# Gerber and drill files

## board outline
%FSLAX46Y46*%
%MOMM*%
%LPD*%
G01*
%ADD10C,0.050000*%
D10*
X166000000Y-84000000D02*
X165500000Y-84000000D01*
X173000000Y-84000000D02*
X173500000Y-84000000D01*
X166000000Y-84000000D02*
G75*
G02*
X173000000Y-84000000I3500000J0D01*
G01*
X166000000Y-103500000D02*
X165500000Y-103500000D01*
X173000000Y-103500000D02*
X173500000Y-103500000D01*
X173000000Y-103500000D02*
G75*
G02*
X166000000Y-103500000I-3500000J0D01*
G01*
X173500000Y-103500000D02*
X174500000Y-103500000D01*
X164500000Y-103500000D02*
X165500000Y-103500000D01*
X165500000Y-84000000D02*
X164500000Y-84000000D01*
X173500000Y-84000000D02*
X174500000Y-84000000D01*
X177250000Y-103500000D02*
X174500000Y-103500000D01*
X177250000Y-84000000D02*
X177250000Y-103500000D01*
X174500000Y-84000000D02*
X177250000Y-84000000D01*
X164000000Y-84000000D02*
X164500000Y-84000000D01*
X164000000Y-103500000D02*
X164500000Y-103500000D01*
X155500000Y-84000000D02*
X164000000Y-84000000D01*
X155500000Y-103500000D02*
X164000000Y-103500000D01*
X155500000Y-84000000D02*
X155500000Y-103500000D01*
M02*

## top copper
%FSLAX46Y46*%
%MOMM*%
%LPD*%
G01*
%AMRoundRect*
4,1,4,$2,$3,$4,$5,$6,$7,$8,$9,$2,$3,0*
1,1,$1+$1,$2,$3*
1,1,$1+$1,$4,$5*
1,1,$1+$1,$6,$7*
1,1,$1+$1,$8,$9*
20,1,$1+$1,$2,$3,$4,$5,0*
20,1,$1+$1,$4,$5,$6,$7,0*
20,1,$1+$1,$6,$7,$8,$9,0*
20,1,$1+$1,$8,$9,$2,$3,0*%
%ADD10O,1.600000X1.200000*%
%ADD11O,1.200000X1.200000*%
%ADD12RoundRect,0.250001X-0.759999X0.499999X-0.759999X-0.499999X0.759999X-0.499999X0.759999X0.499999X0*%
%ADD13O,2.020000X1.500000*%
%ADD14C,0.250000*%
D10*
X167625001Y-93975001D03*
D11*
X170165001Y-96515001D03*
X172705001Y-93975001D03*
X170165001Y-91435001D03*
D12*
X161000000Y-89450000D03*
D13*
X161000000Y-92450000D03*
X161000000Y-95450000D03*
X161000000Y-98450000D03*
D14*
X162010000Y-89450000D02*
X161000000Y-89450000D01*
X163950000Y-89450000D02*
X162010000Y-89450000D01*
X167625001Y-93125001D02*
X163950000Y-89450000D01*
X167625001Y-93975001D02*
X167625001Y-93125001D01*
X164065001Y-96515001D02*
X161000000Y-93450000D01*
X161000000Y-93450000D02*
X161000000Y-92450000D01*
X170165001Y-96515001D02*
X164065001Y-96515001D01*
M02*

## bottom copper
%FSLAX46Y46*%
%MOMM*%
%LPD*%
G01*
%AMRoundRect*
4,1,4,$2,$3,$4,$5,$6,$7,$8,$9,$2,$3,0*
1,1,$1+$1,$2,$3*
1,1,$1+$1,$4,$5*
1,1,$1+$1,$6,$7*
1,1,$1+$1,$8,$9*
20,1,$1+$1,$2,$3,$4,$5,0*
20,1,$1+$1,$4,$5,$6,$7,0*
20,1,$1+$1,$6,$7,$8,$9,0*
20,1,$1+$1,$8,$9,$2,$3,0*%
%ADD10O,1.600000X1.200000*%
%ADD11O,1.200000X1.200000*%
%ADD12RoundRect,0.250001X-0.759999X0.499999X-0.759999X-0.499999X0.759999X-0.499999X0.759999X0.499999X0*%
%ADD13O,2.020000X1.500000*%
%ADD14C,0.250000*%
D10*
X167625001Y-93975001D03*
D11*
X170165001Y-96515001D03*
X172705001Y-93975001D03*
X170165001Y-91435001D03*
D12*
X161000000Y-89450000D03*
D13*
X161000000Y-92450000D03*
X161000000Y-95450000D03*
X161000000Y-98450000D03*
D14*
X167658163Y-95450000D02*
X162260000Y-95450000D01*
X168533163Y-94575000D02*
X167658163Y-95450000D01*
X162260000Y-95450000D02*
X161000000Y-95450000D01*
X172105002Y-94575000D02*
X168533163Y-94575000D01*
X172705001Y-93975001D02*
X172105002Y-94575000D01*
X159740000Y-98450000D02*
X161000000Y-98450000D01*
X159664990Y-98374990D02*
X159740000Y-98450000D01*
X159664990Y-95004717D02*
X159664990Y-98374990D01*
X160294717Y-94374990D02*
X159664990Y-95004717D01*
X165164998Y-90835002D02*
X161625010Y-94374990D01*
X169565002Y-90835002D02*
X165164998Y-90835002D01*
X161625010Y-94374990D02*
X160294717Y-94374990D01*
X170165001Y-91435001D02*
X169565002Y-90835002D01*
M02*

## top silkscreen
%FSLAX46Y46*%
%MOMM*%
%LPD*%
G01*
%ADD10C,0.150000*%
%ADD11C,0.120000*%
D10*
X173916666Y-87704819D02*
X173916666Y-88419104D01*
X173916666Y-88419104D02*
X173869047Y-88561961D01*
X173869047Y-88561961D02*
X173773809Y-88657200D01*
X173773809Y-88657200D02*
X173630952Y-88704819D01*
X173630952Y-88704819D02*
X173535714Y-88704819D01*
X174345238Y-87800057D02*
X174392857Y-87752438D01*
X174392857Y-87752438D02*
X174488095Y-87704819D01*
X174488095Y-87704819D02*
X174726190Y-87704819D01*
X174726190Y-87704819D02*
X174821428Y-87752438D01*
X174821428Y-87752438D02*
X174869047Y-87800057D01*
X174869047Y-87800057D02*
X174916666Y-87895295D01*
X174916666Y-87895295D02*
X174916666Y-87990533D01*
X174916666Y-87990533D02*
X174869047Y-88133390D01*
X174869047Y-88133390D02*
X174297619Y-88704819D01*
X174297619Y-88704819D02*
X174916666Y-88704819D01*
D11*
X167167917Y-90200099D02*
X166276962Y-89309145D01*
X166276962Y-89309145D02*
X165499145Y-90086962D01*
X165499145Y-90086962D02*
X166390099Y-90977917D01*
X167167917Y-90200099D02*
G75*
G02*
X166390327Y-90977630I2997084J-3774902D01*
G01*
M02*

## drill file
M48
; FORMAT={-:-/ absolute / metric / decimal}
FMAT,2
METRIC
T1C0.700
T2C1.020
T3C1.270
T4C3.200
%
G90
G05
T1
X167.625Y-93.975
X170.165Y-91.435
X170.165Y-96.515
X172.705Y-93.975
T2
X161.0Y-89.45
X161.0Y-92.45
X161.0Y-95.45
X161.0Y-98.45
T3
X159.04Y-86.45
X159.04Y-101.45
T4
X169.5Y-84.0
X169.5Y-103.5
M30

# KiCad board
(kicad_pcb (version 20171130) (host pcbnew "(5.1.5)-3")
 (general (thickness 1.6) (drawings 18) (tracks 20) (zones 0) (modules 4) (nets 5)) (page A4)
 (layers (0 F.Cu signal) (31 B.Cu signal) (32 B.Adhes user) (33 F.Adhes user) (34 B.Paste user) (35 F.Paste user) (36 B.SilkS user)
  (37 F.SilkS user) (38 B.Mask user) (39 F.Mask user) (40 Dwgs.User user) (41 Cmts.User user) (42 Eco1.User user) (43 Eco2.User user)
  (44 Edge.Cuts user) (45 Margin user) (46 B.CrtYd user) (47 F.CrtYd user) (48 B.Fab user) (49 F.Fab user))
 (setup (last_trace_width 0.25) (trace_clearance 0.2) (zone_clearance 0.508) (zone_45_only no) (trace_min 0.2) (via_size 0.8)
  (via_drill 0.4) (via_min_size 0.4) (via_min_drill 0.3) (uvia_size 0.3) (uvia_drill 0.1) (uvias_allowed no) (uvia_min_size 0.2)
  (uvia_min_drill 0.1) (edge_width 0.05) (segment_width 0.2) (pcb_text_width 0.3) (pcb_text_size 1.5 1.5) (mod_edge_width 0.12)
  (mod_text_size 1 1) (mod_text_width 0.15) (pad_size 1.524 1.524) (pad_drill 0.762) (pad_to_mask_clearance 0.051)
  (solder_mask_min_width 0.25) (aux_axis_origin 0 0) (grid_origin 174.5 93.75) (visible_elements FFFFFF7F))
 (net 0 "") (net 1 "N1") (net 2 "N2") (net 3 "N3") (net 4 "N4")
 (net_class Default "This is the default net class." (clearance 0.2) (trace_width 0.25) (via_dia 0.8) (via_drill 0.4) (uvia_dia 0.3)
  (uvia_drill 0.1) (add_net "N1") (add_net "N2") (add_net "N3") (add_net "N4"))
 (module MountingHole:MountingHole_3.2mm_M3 (layer F.Cu) (at 169.5 84)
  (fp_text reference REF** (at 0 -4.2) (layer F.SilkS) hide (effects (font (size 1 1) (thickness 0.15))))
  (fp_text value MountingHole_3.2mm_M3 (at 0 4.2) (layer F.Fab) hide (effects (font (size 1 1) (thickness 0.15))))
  (pad 1 np_thru_hole circle (at 0 0) (size 3.2 3.2) (drill 3.2) (layers *.Cu *.Mask)))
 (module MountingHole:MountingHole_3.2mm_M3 (layer F.Cu) (at 169.5 103.5)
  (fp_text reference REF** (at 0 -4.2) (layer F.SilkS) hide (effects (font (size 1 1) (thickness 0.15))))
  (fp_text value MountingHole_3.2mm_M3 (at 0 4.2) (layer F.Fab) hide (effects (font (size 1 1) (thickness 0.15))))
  (pad 1 np_thru_hole circle (at 0 0) (size 3.2 3.2) (drill 3.2) (layers *.Cu *.Mask)))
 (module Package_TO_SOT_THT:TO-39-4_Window (layer F.Cu) (at 167.625001 93.975001)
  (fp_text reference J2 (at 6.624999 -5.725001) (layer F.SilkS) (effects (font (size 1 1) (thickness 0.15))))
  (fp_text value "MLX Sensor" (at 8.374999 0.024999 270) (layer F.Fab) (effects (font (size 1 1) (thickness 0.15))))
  (fp_line (start -0.457084 -3.774902) (end -1.348039 -4.665856) (layer F.SilkS) (width 0.12))
  (fp_line (start -1.348039 -4.665856) (end -2.125856 -3.888039) (layer F.SilkS) (width 0.12))
  (fp_line (start -2.125856 -3.888039) (end -1.234902 -2.997084) (layer F.SilkS) (width 0.12))
  (fp_arc (start 2.54 0) (end -0.457084 -3.774902) (angle 346.9) (layer F.SilkS) (width 0.12))
  (pad 1 thru_hole oval (at 0 0) (size 1.6 1.2) (drill 0.7) (layers *.Cu *.Mask) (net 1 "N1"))
  (pad 2 thru_hole oval (at 2.54 2.54) (size 1.2 1.2) (drill 0.7) (layers *.Cu *.Mask) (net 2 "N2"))
  (pad 3 thru_hole oval (at 5.08 0) (size 1.2 1.2) (drill 0.7) (layers *.Cu *.Mask) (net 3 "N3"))
  (pad 4 thru_hole oval (at 2.54 -2.54) (size 1.2 1.2) (drill 0.7) (layers *.Cu *.Mask) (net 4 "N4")))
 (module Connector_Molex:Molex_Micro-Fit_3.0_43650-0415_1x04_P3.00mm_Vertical (layer B.Cu) (at 161 89.45 270)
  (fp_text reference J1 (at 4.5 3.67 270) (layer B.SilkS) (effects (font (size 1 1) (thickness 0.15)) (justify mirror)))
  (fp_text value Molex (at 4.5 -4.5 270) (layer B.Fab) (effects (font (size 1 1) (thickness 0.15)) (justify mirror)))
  (pad "" np_thru_hole circle (at -3 1.96 270) (size 1.27 1.27) (drill 1.27) (layers *.Cu *.Mask))
  (pad "" np_thru_hole circle (at 12 1.96 270) (size 1.27 1.27) (drill 1.27) (layers *.Cu *.Mask))
  (pad 1 thru_hole roundrect (at 0 0 270) (size 1.5 2.02) (drill 1.02) (layers *.Cu *.Mask) (roundrect_rratio 0.166667) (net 1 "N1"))
  (pad 2 thru_hole oval (at 3 0 270) (size 1.5 2.02) (drill 1.02) (layers *.Cu *.Mask) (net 2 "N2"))
  (pad 3 thru_hole oval (at 6 0 270) (size 1.5 2.02) (drill 1.02) (layers *.Cu *.Mask) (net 3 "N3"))
  (pad 4 thru_hole oval (at 9 0 270) (size 1.5 2.02) (drill 1.02) (layers *.Cu *.Mask) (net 4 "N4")))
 (gr_line (start 166 84) (end 165.5 84) (layer Edge.Cuts) (width 0.05))
 (gr_line (start 173 84) (end 173.5 84) (layer Edge.Cuts) (width 0.05))
 (gr_arc (start 169.5 84) (end 173 84) (angle -180) (layer Edge.Cuts) (width 0.05))
 (gr_line (start 166 103.5) (end 165.5 103.5) (layer Edge.Cuts) (width 0.05))
 (gr_line (start 173 103.5) (end 173.5 103.5) (layer Edge.Cuts) (width 0.05))
 (gr_arc (start 169.5 103.5) (end 166 103.5) (angle -180) (layer Edge.Cuts) (width 0.05))
 (gr_line (start 173.5 103.5) (end 174.5 103.5) (layer Edge.Cuts) (width 0.05))
 (gr_line (start 164.5 103.5) (end 165.5 103.5) (layer Edge.Cuts) (width 0.05))
 (gr_line (start 165.5 84) (end 164.5 84) (layer Edge.Cuts) (width 0.05))
 (gr_line (start 173.5 84) (end 174.5 84) (layer Edge.Cuts) (width 0.05))
 (gr_line (start 177.25 103.5) (end 174.5 103.5) (layer Edge.Cuts) (width 0.05))
 (gr_line (start 177.25 84) (end 177.25 103.5) (layer Edge.Cuts) (width 0.05))
 (gr_line (start 174.5 84) (end 177.25 84) (layer Edge.Cuts) (width 0.05))
 (gr_line (start 164 84) (end 164.5 84) (layer Edge.Cuts) (width 0.05))
 (gr_line (start 164 103.5) (end 164.5 103.5) (layer Edge.Cuts) (width 0.05))
 (gr_line (start 155.5 84) (end 164 84) (layer Edge.Cuts) (width 0.05))
 (gr_line (start 155.5 103.5) (end 164 103.5) (layer Edge.Cuts) (width 0.05))
 (gr_line (start 155.5 84) (end 155.5 103.5) (layer Edge.Cuts) (width 0.05))
 (segment (start 162.01 89.45) (end 161 89.45) (width 0.25) (layer F.Cu) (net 1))
 (segment (start 163.95 89.45) (end 162.01 89.45) (width 0.25) (layer F.Cu) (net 1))
 (segment (start 167.625001 93.125001) (end 163.95 89.45) (width 0.25) (layer F.Cu) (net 1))
 (segment (start 167.625001 93.975001) (end 167.625001 93.125001) (width 0.25) (layer F.Cu) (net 1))
 (segment (start 164.065001 96.515001) (end 161 93.45) (width 0.25) (layer F.Cu) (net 2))
 (segment (start 161 93.45) (end 161 92.45) (width 0.25) (layer F.Cu) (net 2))
 (segment (start 170.165001 96.515001) (end 164.065001 96.515001) (width 0.25) (layer F.Cu) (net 2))
 (segment (start 167.658163 95.45) (end 162.26 95.45) (width 0.25) (layer B.Cu) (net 3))
 (segment (start 168.533163 94.575) (end 167.658163 95.45) (width 0.25) (layer B.Cu) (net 3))
 (segment (start 162.26 95.45) (end 161 95.45) (width 0.25) (layer B.Cu) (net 3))
 (segment (start 172.105002 94.575) (end 168.533163 94.575) (width 0.25) (layer B.Cu) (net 3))
 (segment (start 172.705001 93.975001) (end 172.105002 94.575) (width 0.25) (layer B.Cu) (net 3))
 (segment (start 159.74 98.45) (end 161 98.45) (width 0.25) (layer B.Cu) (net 4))
 (segment (start 159.66499 98.37499) (end 159.74 98.45) (width 0.25) (layer B.Cu) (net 4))
 (segment (start 159.66499 95.004717) (end 159.66499 98.37499) (width 0.25) (layer B.Cu) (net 4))
 (segment (start 160.294717 94.37499) (end 159.66499 95.004717) (width 0.25) (layer B.Cu) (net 4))
 (segment (start 165.164998 90.835002) (end 161.62501 94.37499) (width 0.25) (layer B.Cu) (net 4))
 (segment (start 169.565002 90.835002) (end 165.164998 90.835002) (width 0.25) (layer B.Cu) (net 4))
 (segment (start 161.62501 94.37499) (end 160.294717 94.37499) (width 0.25) (layer B.Cu) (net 4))
 (segment (start 170.165001 91.435001) (end 169.565002 90.835002) (width 0.25) (layer B.Cu) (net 4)))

